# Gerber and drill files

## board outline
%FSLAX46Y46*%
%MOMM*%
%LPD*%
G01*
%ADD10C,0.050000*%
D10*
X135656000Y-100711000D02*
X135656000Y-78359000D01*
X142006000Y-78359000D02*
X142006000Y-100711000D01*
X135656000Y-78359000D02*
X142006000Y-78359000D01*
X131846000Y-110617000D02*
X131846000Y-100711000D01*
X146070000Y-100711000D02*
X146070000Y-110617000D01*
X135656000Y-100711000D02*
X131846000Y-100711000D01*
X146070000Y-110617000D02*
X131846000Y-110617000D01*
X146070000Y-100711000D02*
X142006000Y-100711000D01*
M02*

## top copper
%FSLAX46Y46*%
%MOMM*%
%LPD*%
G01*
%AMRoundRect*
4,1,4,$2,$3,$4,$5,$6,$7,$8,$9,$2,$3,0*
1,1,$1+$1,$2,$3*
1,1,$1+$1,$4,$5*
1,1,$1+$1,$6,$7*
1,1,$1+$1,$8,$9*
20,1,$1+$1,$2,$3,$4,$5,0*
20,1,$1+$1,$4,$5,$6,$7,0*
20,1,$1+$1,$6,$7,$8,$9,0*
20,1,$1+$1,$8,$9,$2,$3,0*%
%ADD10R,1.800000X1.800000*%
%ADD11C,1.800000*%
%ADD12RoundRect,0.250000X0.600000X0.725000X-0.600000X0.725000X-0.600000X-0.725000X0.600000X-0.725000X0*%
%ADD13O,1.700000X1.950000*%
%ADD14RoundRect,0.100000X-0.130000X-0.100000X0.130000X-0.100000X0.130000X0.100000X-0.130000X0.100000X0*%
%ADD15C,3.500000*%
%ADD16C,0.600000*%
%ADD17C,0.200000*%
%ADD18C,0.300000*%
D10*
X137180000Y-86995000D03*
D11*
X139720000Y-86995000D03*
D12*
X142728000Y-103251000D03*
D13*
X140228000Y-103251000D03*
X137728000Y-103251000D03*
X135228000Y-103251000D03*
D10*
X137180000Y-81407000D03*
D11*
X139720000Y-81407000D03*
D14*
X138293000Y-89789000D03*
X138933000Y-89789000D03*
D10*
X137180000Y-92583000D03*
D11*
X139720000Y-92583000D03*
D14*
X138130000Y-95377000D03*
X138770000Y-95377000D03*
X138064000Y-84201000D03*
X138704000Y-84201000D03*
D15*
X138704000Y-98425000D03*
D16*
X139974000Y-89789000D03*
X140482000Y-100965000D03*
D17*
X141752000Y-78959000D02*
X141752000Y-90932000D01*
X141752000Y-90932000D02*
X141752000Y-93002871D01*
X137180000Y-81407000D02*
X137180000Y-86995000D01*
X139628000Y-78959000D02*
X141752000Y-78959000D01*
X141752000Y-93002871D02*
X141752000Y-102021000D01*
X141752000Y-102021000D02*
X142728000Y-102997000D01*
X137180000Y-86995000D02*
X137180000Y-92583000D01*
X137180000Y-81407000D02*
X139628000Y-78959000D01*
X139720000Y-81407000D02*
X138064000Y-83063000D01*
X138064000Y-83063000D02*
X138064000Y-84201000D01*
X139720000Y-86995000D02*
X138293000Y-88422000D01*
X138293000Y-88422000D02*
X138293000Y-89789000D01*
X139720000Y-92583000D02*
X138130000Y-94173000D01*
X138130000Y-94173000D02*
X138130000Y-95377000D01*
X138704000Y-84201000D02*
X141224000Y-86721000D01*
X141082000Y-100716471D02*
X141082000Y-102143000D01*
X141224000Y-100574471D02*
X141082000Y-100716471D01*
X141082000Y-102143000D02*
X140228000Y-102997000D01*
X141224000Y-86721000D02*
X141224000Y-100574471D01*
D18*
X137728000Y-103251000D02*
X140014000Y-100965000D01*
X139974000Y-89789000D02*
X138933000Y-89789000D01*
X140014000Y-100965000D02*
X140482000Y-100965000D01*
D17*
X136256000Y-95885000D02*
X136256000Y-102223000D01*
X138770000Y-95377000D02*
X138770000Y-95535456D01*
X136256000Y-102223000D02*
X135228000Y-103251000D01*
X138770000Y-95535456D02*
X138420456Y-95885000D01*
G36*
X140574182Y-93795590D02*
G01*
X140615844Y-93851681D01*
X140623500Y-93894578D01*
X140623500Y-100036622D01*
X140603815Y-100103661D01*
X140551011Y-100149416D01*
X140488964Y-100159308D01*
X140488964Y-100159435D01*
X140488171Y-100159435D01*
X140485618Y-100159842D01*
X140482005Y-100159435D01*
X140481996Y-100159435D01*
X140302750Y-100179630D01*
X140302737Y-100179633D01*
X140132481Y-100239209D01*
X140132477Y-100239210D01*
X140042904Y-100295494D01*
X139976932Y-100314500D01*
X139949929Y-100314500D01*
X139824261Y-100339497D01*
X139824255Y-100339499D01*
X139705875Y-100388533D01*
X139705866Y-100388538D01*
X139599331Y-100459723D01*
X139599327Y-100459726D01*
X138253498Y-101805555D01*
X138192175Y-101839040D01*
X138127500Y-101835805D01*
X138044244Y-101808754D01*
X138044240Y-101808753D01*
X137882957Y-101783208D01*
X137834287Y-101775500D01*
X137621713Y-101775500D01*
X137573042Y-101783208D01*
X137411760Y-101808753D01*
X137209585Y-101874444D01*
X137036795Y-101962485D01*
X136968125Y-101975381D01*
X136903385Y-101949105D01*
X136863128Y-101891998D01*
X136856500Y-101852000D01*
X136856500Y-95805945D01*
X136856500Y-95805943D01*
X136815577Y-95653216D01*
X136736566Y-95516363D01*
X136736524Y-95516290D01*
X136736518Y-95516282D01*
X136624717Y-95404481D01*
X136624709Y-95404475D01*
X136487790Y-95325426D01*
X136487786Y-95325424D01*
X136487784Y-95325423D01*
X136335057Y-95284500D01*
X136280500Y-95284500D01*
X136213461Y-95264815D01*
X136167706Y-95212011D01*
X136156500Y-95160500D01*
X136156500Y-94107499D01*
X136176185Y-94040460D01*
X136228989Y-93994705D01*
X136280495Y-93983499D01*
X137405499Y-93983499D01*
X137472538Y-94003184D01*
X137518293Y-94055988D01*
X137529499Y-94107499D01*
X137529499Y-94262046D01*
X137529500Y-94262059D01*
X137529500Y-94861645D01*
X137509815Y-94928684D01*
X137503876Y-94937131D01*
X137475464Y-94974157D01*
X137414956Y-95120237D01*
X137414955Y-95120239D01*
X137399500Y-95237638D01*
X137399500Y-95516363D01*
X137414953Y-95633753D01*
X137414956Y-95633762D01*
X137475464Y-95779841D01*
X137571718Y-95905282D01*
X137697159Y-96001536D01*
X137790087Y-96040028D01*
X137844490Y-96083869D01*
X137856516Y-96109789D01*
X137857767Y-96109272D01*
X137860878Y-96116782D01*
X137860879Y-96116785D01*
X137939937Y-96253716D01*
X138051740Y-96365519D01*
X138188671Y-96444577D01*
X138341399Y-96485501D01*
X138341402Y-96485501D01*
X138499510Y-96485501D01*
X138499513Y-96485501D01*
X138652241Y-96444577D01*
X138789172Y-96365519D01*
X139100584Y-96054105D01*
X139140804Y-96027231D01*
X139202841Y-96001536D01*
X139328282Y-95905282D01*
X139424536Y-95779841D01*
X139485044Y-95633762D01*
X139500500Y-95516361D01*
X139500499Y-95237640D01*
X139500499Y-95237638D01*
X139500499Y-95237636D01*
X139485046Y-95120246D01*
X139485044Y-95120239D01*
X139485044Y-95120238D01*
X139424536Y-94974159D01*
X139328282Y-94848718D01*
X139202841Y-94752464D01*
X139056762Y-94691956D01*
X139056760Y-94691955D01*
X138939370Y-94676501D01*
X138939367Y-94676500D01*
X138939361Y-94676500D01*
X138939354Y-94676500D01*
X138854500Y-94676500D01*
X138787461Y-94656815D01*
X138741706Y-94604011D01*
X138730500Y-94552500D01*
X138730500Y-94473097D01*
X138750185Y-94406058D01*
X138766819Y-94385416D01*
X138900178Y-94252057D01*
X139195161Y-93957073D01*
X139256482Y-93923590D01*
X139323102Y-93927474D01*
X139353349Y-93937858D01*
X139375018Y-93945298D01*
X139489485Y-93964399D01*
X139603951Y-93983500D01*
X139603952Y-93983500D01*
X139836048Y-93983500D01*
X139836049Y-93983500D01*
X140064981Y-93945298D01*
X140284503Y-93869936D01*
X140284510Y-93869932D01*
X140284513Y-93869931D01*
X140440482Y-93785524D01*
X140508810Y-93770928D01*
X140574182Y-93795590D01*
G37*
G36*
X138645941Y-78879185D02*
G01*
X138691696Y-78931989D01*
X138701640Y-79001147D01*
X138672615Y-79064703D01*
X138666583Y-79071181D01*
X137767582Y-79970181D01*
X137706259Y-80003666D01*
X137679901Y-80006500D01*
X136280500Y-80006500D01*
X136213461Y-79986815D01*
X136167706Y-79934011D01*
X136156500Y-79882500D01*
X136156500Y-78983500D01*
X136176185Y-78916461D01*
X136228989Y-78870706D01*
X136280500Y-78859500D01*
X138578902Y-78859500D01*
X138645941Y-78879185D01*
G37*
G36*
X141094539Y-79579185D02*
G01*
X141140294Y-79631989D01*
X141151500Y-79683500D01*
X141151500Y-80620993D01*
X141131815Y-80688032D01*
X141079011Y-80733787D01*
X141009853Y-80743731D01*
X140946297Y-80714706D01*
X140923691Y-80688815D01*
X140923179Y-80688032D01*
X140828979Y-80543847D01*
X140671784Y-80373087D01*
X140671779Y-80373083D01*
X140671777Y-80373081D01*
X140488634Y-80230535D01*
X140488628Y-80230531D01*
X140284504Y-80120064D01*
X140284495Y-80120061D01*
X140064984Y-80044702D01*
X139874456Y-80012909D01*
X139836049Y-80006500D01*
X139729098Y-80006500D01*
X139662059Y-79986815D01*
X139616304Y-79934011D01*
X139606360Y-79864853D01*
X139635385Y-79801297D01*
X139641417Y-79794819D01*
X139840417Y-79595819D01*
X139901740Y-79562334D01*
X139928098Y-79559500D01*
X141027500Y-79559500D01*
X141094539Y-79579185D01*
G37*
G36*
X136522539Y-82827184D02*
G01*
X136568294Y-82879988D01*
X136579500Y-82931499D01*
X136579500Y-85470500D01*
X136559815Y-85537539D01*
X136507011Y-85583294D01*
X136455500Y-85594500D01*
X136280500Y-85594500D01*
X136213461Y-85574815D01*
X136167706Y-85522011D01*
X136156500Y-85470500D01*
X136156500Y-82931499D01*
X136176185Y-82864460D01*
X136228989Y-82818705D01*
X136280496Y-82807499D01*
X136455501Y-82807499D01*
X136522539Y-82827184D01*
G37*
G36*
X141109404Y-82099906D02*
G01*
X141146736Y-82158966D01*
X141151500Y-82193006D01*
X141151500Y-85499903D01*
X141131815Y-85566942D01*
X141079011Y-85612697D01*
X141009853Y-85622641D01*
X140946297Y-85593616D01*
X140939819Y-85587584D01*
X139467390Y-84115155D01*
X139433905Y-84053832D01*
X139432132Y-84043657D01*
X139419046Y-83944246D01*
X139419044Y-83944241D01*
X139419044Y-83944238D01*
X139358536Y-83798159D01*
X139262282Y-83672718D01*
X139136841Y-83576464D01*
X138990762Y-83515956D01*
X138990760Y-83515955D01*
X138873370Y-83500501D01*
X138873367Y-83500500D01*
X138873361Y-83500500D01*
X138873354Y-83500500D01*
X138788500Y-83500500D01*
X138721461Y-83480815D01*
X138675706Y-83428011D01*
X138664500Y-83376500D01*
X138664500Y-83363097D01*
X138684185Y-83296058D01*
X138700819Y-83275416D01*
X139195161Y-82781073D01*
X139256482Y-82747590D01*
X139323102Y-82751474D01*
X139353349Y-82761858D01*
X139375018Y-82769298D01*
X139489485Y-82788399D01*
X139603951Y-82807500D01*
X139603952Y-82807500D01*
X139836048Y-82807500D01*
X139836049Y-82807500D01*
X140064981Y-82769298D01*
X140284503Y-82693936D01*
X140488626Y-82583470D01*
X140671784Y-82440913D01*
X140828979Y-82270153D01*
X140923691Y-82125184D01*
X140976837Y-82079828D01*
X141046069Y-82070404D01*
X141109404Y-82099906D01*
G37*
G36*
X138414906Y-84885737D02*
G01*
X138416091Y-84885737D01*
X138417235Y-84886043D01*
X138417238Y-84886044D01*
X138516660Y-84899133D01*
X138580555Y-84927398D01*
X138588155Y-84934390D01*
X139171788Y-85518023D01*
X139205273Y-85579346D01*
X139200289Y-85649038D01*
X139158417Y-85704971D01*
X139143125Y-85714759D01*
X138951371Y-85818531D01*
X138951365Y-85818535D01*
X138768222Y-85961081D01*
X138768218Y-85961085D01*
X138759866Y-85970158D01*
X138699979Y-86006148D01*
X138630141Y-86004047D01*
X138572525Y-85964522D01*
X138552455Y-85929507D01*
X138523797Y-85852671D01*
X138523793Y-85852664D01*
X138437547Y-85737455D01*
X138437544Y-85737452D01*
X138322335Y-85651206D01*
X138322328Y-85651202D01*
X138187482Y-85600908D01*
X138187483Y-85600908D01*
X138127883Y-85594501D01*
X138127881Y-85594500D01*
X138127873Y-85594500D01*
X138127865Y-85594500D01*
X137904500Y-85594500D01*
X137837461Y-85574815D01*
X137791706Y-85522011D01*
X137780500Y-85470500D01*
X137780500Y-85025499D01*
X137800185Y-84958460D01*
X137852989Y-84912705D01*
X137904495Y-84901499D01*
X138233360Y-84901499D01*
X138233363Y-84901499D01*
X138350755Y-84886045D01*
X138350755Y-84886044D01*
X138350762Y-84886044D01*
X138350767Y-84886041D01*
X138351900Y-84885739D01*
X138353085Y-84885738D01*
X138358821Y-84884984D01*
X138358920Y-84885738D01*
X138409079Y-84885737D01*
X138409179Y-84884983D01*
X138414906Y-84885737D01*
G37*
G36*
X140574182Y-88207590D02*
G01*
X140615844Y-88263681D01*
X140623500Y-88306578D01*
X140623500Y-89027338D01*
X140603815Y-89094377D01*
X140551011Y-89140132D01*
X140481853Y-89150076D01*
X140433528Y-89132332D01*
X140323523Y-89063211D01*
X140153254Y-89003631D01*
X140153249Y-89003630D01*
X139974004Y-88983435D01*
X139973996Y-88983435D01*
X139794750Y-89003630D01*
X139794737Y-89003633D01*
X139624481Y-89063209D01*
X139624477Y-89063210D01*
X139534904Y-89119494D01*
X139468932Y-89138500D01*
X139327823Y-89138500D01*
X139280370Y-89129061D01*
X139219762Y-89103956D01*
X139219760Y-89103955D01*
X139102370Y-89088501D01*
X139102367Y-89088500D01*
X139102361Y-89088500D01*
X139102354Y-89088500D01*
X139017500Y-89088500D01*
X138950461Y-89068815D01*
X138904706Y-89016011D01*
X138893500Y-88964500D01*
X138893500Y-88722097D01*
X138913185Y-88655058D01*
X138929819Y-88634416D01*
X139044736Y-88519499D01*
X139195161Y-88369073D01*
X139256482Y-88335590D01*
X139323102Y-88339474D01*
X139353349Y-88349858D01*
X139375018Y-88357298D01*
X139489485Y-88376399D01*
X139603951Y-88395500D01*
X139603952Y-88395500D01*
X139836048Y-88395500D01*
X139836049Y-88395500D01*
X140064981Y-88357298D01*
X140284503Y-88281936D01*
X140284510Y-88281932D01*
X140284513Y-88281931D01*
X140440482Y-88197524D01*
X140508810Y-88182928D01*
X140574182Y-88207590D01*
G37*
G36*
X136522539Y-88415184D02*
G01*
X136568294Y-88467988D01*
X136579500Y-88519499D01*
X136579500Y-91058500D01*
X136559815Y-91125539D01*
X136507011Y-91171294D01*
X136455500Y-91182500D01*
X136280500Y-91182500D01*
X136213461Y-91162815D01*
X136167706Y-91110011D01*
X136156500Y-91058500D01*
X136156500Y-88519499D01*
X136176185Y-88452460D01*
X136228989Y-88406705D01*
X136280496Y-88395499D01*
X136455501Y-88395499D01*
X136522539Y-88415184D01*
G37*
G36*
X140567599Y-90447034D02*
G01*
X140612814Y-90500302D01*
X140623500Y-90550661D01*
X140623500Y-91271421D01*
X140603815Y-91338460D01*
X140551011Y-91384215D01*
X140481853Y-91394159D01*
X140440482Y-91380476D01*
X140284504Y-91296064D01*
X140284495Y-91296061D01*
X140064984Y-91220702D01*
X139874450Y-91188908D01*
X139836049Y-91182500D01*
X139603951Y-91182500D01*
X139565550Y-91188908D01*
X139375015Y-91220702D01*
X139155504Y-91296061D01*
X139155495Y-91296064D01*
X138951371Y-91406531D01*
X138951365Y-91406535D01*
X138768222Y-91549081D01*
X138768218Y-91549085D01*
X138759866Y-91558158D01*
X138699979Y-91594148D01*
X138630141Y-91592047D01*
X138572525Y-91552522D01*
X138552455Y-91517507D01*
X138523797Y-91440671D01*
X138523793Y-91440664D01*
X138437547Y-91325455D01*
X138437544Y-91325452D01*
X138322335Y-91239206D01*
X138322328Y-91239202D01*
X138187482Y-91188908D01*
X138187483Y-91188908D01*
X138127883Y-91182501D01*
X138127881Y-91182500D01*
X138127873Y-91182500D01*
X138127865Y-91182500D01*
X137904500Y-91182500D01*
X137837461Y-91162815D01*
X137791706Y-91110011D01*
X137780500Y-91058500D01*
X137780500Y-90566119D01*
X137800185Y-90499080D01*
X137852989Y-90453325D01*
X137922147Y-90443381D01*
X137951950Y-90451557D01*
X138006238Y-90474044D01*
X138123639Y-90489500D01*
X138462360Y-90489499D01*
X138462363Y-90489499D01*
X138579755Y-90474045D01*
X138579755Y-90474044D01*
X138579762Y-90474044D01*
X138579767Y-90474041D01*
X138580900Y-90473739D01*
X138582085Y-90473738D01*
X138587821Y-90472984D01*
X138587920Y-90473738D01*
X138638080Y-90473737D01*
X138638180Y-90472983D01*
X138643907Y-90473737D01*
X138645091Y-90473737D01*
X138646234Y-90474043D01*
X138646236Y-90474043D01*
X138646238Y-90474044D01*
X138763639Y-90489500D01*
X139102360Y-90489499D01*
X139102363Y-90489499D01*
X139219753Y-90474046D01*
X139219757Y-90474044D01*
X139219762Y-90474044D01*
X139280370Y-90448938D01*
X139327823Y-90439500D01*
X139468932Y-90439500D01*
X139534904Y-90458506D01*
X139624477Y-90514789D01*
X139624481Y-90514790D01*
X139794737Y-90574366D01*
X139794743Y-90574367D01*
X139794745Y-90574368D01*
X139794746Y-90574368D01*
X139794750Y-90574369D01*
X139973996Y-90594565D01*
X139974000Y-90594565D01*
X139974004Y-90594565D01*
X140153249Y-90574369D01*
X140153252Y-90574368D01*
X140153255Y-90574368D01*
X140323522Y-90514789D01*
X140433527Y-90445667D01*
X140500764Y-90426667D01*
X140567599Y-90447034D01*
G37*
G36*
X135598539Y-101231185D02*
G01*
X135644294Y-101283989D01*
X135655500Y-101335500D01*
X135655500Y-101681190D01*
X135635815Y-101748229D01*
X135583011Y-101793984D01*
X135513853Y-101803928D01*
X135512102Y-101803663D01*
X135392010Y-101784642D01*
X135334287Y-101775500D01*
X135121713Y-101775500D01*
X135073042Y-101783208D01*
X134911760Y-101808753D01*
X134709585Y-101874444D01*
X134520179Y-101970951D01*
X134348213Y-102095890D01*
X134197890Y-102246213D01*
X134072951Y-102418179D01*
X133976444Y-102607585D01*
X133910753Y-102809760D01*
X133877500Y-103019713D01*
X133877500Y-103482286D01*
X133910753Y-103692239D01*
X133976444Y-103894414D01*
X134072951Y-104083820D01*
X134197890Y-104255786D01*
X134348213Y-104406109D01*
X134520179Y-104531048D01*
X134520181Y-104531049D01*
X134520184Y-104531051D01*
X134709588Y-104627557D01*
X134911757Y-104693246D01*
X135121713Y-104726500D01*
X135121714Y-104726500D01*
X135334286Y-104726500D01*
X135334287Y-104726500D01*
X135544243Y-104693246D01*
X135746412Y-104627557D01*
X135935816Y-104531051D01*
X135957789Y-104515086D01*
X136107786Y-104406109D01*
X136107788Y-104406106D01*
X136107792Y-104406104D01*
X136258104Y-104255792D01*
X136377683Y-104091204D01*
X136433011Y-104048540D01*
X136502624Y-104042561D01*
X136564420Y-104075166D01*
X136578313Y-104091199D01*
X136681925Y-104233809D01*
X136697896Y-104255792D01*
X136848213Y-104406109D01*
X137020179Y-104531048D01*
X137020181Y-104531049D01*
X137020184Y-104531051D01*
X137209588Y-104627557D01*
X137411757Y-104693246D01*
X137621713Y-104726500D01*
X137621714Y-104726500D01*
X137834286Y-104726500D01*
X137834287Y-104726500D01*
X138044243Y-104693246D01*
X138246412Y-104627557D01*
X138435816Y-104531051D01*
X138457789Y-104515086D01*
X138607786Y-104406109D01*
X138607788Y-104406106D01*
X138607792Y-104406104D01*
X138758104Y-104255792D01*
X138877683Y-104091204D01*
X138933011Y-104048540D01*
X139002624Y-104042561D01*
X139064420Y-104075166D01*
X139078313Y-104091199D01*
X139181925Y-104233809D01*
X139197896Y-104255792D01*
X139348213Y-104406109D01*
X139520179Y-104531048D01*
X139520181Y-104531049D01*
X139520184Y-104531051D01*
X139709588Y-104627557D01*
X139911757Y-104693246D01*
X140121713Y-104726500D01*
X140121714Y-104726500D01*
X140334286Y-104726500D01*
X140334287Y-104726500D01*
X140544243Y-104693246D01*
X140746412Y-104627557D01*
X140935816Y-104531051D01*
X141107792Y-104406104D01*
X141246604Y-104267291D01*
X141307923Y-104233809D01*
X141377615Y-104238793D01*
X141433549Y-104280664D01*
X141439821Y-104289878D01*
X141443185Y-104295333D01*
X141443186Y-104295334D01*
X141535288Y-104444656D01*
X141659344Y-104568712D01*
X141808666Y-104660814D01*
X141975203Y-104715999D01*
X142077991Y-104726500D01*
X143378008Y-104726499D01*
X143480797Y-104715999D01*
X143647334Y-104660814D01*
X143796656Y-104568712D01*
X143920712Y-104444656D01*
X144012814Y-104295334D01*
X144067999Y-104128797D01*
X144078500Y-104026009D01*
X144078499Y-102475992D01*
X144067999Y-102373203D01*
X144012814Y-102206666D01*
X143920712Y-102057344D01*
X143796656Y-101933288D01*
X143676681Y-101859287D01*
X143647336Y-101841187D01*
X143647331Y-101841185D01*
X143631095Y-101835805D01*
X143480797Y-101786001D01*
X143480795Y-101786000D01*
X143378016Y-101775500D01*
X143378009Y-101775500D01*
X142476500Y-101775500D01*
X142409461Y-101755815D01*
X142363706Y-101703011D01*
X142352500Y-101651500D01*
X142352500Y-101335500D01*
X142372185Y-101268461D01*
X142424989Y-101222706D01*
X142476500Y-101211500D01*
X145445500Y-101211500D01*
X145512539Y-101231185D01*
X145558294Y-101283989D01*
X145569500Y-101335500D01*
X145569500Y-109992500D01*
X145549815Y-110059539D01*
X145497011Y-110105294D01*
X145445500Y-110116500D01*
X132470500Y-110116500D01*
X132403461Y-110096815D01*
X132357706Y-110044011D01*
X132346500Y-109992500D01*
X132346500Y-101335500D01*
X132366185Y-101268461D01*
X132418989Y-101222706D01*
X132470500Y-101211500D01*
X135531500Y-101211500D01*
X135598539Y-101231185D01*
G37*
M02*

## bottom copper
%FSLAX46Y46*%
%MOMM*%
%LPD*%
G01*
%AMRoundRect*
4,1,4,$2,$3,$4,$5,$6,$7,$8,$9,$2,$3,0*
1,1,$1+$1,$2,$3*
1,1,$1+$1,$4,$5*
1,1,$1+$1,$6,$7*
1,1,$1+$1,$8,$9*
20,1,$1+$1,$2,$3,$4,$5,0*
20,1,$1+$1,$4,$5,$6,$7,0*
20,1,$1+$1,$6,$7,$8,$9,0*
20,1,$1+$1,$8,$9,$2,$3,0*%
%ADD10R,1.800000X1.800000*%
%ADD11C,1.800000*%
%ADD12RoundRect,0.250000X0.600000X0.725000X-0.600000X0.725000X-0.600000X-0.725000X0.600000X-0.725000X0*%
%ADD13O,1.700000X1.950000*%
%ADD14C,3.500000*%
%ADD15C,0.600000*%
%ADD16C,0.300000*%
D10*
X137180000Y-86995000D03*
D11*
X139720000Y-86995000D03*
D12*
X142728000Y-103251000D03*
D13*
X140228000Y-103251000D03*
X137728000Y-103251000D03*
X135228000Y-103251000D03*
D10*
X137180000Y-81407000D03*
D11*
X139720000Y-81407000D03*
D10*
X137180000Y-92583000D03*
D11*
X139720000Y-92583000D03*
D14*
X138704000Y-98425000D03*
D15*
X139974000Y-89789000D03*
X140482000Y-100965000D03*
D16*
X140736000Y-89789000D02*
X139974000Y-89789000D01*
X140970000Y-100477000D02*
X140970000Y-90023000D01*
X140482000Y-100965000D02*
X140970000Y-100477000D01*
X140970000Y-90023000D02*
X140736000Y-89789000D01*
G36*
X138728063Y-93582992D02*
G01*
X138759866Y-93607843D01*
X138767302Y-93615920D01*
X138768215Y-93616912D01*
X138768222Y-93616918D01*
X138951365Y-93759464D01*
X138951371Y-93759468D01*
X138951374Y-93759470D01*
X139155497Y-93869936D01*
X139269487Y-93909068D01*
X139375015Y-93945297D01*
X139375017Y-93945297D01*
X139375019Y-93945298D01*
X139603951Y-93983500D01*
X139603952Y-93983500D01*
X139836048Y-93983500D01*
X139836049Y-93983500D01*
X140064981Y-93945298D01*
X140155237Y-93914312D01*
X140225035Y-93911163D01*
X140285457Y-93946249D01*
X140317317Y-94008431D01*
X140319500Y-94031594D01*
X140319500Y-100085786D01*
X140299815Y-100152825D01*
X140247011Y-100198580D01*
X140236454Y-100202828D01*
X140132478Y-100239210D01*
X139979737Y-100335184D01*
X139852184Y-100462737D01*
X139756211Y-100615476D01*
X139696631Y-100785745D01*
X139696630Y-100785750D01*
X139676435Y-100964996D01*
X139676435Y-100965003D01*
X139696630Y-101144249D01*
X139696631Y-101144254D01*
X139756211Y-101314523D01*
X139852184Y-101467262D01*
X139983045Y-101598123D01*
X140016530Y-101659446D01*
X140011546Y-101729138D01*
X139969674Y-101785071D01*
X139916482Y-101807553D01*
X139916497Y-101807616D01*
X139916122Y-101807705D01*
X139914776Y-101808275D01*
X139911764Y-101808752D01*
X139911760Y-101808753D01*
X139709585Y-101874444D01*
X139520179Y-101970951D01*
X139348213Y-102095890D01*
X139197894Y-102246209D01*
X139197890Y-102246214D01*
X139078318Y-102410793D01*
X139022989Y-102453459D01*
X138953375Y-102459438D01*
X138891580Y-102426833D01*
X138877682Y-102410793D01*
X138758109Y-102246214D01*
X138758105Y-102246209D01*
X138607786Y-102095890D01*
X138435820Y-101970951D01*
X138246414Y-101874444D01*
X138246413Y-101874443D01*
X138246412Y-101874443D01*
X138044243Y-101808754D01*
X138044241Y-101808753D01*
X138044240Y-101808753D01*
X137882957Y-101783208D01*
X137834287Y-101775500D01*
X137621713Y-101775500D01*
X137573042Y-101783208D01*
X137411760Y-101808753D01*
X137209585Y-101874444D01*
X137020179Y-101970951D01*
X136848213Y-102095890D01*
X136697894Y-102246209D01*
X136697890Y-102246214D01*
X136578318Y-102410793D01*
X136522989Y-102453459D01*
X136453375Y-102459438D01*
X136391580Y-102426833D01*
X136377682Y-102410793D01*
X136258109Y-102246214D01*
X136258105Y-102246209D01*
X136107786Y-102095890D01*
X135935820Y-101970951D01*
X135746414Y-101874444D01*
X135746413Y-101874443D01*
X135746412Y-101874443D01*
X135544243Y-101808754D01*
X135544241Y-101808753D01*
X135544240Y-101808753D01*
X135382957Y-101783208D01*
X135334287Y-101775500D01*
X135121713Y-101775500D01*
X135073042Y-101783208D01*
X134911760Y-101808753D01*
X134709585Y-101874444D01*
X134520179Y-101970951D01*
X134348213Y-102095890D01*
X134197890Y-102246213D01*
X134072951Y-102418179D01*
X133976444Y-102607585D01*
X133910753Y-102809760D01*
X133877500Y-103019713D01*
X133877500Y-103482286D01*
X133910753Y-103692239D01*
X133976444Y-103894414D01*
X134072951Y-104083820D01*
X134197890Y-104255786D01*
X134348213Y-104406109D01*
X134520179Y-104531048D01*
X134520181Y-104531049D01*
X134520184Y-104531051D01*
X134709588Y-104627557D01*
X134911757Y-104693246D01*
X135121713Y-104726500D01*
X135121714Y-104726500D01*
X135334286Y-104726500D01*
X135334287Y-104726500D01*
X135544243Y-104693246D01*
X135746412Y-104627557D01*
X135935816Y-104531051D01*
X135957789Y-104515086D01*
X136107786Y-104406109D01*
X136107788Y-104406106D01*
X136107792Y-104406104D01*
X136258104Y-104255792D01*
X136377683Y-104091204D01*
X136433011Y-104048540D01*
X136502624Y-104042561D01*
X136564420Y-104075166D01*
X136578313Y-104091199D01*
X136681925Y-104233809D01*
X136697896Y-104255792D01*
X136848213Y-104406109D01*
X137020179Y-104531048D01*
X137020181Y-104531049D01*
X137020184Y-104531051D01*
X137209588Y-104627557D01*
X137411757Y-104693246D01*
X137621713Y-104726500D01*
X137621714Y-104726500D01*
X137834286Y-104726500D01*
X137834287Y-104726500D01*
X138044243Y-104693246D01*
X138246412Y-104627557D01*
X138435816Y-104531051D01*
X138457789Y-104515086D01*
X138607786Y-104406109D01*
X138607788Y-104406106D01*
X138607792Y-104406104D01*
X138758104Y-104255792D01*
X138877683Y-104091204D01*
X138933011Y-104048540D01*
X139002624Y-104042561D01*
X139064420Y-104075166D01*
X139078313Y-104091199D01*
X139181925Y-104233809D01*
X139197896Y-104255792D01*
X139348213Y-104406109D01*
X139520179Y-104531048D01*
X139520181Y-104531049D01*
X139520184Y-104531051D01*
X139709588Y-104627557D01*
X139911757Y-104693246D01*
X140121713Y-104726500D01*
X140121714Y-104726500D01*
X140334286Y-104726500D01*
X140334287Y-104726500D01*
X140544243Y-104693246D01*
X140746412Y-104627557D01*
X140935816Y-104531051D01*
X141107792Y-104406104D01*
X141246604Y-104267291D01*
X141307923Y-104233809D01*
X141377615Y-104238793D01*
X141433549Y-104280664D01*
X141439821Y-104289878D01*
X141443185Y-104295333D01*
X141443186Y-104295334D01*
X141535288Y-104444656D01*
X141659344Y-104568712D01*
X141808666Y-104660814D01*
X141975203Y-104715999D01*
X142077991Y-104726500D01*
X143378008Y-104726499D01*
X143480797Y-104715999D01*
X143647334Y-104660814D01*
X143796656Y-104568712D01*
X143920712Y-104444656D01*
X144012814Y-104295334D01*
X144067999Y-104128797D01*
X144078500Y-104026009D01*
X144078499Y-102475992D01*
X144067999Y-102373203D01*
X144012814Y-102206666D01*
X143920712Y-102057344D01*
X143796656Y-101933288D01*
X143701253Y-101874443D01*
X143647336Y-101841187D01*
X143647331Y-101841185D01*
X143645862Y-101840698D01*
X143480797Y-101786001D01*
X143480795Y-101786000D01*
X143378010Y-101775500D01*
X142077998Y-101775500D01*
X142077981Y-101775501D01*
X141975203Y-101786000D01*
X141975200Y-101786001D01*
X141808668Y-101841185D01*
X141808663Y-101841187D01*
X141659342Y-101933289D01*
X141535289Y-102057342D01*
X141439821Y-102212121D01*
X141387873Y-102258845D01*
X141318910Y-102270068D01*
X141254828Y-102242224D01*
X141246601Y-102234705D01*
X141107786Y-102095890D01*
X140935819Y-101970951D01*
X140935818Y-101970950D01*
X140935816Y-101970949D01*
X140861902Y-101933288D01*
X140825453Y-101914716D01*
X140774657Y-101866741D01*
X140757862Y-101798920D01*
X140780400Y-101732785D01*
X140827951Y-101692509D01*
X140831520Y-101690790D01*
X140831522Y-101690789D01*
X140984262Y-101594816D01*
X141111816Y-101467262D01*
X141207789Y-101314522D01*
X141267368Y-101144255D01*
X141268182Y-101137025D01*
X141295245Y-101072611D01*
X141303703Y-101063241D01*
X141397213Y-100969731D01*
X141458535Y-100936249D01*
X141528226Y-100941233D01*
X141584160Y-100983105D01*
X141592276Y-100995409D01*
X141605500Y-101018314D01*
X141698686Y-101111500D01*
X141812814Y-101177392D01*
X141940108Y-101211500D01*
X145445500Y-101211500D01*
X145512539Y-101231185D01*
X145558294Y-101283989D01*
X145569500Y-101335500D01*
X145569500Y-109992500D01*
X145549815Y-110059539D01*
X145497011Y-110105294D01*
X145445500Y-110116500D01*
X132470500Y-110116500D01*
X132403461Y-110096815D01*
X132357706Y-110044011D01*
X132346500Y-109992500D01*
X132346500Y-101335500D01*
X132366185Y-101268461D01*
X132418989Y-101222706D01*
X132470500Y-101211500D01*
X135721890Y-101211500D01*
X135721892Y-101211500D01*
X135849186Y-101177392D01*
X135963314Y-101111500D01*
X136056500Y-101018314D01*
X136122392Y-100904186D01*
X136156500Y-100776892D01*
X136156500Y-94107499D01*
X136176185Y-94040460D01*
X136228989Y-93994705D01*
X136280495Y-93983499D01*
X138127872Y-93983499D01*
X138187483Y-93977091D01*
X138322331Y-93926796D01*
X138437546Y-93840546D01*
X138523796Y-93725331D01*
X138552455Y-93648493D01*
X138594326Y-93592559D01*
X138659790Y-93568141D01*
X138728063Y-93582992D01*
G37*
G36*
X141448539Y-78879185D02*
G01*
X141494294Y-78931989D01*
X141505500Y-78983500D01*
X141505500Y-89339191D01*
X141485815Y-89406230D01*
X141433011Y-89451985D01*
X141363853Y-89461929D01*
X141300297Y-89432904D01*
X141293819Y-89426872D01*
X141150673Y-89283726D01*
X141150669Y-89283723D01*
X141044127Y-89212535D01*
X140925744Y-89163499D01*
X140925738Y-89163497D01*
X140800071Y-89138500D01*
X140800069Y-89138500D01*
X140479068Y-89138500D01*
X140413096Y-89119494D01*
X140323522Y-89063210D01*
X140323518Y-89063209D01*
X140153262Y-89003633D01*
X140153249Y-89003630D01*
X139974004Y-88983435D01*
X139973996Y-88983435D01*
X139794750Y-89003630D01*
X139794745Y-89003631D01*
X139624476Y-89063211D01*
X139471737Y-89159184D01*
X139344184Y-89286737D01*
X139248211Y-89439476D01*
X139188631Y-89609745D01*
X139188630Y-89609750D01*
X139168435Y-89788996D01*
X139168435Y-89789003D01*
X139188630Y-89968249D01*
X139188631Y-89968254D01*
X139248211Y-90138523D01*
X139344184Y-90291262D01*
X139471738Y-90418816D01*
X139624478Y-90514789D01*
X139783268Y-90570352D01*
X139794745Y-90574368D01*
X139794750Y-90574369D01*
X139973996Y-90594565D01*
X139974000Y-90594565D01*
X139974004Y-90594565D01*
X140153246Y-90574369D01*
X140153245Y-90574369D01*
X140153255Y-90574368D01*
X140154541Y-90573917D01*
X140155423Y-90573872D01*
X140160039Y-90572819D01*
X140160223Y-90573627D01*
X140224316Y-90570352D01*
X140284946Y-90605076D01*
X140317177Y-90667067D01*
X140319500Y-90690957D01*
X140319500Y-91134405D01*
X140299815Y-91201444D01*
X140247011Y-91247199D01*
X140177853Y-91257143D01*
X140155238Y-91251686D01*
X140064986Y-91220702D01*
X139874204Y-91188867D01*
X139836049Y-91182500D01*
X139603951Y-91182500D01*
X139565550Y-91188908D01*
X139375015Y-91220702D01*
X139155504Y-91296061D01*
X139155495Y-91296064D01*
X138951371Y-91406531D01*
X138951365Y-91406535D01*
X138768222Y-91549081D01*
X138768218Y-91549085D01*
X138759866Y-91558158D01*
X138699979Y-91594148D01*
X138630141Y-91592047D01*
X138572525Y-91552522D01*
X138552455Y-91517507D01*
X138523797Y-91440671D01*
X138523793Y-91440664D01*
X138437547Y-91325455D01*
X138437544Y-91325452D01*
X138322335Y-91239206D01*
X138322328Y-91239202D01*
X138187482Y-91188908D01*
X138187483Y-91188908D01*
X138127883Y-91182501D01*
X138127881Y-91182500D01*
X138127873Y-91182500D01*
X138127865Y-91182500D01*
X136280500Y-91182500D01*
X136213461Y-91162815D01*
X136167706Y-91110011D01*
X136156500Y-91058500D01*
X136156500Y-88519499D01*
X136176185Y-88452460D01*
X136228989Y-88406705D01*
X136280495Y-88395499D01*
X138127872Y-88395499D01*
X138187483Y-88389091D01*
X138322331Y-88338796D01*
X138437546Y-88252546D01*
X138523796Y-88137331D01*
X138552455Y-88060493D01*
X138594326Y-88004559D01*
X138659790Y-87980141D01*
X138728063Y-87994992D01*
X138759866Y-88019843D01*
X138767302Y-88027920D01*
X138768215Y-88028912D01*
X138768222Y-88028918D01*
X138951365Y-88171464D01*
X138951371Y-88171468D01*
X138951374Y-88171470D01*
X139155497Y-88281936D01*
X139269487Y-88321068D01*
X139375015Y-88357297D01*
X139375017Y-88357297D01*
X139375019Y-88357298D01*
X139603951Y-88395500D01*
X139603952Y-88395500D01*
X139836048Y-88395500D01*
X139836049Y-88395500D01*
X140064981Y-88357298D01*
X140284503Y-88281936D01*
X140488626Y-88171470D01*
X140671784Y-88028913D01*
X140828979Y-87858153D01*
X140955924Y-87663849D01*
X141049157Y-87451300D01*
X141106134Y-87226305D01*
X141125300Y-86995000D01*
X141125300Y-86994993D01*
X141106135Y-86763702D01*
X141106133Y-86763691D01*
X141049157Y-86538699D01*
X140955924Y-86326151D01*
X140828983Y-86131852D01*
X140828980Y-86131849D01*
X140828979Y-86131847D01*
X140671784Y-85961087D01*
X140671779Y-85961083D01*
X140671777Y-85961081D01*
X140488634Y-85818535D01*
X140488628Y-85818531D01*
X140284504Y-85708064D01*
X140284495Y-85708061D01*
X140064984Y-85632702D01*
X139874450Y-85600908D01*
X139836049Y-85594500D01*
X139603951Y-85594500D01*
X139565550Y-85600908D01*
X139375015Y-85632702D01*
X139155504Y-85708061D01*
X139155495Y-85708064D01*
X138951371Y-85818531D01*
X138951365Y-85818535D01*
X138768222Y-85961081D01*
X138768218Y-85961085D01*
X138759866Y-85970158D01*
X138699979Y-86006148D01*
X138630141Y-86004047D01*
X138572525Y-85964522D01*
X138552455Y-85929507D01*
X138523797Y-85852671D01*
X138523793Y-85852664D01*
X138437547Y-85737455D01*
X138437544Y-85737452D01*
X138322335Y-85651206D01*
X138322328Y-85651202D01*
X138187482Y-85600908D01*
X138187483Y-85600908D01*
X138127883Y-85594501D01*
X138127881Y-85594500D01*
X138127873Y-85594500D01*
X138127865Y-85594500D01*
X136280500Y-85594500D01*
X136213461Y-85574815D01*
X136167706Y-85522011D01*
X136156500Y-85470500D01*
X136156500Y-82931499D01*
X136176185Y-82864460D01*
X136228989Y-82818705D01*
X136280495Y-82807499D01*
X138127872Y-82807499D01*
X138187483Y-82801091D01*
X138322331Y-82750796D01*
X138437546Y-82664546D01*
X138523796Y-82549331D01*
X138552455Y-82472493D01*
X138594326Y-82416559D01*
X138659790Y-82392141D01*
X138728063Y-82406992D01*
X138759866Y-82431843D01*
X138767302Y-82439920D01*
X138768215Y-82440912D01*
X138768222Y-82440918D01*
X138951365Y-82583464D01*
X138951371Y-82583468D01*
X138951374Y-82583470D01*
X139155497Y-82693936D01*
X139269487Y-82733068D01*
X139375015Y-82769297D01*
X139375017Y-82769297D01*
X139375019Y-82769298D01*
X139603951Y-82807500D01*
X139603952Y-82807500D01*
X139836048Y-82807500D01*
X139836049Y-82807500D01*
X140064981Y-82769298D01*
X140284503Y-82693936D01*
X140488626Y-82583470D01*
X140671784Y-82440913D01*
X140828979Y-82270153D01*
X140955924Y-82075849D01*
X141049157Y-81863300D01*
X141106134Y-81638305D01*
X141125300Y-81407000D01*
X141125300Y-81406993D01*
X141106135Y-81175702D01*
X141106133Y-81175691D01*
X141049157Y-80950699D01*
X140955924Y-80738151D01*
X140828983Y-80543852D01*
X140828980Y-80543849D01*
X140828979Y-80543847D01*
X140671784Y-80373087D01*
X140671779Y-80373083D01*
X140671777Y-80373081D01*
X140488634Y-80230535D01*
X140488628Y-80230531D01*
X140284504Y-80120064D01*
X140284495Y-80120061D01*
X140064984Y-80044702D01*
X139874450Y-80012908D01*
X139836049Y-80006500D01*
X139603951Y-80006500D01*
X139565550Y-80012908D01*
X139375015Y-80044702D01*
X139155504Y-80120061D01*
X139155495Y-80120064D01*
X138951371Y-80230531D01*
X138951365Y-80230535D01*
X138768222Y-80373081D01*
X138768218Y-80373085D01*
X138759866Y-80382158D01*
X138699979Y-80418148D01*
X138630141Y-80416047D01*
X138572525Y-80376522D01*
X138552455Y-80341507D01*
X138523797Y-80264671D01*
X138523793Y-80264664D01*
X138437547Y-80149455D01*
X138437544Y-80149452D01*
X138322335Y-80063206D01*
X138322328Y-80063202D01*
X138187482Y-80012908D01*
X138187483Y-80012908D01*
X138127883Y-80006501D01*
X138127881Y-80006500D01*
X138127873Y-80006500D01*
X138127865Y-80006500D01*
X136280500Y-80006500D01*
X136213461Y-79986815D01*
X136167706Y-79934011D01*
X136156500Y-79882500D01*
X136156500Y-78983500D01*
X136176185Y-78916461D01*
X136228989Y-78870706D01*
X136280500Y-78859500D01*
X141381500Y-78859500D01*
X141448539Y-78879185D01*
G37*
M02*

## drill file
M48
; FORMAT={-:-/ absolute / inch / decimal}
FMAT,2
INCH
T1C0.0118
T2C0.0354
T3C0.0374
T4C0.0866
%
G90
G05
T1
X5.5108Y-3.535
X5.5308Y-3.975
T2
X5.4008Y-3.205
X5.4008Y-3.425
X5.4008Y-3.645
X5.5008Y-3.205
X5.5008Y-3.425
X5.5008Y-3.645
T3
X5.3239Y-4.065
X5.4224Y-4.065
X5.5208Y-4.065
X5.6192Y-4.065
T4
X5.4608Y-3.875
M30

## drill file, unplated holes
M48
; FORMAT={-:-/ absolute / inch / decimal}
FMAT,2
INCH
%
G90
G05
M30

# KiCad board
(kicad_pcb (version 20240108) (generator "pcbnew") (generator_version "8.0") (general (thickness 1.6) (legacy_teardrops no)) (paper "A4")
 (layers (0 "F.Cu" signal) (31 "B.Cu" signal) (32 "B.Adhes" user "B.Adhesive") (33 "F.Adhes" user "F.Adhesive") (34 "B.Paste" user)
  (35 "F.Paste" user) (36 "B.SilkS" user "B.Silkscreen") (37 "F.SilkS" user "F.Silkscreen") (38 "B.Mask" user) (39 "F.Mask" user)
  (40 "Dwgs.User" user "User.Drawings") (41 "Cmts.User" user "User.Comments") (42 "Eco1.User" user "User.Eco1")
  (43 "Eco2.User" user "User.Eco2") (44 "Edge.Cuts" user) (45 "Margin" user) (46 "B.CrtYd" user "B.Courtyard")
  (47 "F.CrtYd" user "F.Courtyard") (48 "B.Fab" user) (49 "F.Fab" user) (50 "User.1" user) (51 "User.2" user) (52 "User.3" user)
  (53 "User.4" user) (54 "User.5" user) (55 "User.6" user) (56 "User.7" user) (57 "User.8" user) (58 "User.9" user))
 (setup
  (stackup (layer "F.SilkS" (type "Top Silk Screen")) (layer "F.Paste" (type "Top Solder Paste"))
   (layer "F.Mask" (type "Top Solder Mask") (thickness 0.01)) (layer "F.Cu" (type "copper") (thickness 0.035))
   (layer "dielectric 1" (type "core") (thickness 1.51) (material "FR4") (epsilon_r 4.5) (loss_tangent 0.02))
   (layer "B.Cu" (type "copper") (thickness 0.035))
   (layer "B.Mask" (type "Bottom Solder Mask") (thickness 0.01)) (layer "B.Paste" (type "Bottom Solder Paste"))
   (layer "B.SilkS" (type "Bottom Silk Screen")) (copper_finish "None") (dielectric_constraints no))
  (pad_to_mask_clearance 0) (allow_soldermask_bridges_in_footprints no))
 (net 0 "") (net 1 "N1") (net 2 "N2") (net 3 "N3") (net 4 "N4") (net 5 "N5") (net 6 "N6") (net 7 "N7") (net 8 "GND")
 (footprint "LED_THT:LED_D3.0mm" (layer "F.Cu") (at 137.18 86.995)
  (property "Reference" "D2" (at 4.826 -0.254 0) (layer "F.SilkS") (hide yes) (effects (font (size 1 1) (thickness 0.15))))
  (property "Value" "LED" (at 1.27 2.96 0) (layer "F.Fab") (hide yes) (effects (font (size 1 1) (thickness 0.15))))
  (pad "1" thru_hole rect (at 0 0) (size 1.8 1.8) (drill 0.9) (layers "*.Cu" "*.Mask") (remove_unused_layers no) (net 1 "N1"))
  (pad "2" thru_hole circle (at 2.54 0) (size 1.8 1.8) (drill 0.9) (layers "*.Cu" "*.Mask") (remove_unused_layers no) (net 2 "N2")))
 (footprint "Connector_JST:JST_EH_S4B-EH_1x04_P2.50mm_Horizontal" (layer "F.Cu") (at 142.728 103.251 180)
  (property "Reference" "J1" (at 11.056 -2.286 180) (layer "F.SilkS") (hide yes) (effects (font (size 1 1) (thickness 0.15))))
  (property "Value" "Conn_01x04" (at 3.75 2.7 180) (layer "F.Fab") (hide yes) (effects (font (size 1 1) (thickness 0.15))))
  (pad "1" thru_hole roundrect (at 0 0 180) (size 1.7 1.95) (drill 0.95) (layers "*.Cu" "*.Mask") (remove_unused_layers no)
   (roundrect_rratio 0.147059) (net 1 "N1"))
  (pad "2" thru_hole oval (at 2.5 0 180) (size 1.7 1.95) (drill 0.95) (layers "*.Cu" "*.Mask") (remove_unused_layers no) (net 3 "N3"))
  (pad "3" thru_hole oval (at 5 0 180) (size 1.7 1.95) (drill 0.95) (layers "*.Cu" "*.Mask") (remove_unused_layers no) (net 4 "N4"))
  (pad "4" thru_hole oval (at 7.5 0 180) (size 1.7 1.95) (drill 0.95) (layers "*.Cu" "*.Mask") (remove_unused_layers no) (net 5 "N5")))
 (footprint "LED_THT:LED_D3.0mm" (layer "F.Cu") (at 137.18 81.407)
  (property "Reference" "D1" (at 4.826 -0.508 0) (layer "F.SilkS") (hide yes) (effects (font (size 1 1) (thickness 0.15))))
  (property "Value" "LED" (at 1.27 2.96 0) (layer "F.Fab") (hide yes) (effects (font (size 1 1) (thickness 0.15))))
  (pad "1" thru_hole rect (at 0 0) (size 1.8 1.8) (drill 0.9) (layers "*.Cu" "*.Mask") (remove_unused_layers no) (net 1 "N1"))
  (pad "2" thru_hole circle (at 2.54 0) (size 1.8 1.8) (drill 0.9) (layers "*.Cu" "*.Mask") (remove_unused_layers no) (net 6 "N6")))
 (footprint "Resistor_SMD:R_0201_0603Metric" (layer "F.Cu") (at 138.613 89.789)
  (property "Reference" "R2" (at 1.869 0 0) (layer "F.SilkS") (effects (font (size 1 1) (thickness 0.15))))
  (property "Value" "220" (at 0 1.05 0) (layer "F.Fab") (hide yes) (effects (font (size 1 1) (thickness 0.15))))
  (pad "" smd roundrect (at -0.345 0) (size 0.318 0.36) (layers "F.Paste") (roundrect_rratio 0.25))
  (pad "" smd roundrect (at 0.345 0) (size 0.318 0.36) (layers "F.Paste") (roundrect_rratio 0.25))
  (pad "1" smd roundrect (at -0.32 0) (size 0.46 0.4) (layers "F.Cu" "F.Mask") (roundrect_rratio 0.25) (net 2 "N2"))
  (pad "2" smd roundrect (at 0.32 0) (size 0.46 0.4) (layers "F.Cu" "F.Mask") (roundrect_rratio 0.25) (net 4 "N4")))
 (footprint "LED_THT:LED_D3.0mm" (layer "F.Cu") (at 137.18 92.583)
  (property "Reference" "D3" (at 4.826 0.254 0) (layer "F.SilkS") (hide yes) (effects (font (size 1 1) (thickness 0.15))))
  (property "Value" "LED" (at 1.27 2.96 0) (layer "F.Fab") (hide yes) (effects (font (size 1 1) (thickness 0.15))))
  (pad "1" thru_hole rect (at 0 0) (size 1.8 1.8) (drill 0.9) (layers "*.Cu" "*.Mask") (remove_unused_layers no) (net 1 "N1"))
  (pad "2" thru_hole circle (at 2.54 0) (size 1.8 1.8) (drill 0.9) (layers "*.Cu" "*.Mask") (remove_unused_layers no) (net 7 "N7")))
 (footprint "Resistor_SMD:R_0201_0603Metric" (layer "F.Cu") (at 138.45 95.377)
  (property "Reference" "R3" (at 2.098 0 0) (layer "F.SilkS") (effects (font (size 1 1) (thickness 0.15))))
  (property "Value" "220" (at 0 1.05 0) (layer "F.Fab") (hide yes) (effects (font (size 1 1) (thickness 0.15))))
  (pad "" smd roundrect (at -0.345 0) (size 0.318 0.36) (layers "F.Paste") (roundrect_rratio 0.25))
  (pad "" smd roundrect (at 0.345 0) (size 0.318 0.36) (layers "F.Paste") (roundrect_rratio 0.25))
  (pad "1" smd roundrect (at -0.32 0) (size 0.46 0.4) (layers "F.Cu" "F.Mask") (roundrect_rratio 0.25) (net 7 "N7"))
  (pad "2" smd roundrect (at 0.32 0) (size 0.46 0.4) (layers "F.Cu" "F.Mask") (roundrect_rratio 0.25) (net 5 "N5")))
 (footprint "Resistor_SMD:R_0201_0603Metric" (layer "F.Cu") (at 138.384 84.201)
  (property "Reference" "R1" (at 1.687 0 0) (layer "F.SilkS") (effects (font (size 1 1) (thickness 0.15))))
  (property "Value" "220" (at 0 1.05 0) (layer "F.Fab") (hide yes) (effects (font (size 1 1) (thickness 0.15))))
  (pad "" smd roundrect (at -0.345 0) (size 0.318 0.36) (layers "F.Paste") (roundrect_rratio 0.25))
  (pad "" smd roundrect (at 0.345 0) (size 0.318 0.36) (layers "F.Paste") (roundrect_rratio 0.25))
  (pad "1" smd roundrect (at -0.32 0) (size 0.46 0.4) (layers "F.Cu" "F.Mask") (roundrect_rratio 0.25) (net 6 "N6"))
  (pad "2" smd roundrect (at 0.32 0) (size 0.46 0.4) (layers "F.Cu" "F.Mask") (roundrect_rratio 0.25) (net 3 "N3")))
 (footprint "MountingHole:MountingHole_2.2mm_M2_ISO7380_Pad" (layer "F.Cu") (at 138.704 98.425)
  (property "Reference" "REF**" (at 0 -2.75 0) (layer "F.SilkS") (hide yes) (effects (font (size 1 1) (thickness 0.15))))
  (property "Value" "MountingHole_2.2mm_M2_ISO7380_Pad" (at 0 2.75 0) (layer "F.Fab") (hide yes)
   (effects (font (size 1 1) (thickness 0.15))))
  (pad "1" thru_hole circle (at 0 0) (size 3.5 3.5) (drill 2.2) (layers "*.Cu" "*.Mask") (remove_unused_layers no) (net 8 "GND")))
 (gr_line (start 135.656 100.711) (end 135.656 78.359) (stroke (width 0.05) (type default)) (layer "Edge.Cuts"))
 (gr_line (start 142.006 78.359) (end 142.006 100.711) (stroke (width 0.05) (type default)) (layer "Edge.Cuts"))
 (gr_line (start 135.656 78.359) (end 142.006 78.359) (stroke (width 0.05) (type default)) (layer "Edge.Cuts"))
 (gr_line (start 131.846 110.617) (end 131.846 100.711) (stroke (width 0.05) (type default)) (layer "Edge.Cuts"))
 (gr_line (start 146.07 100.711) (end 146.07 110.617) (stroke (width 0.05) (type default)) (layer "Edge.Cuts"))
 (gr_line (start 135.656 100.711) (end 131.846 100.711) (stroke (width 0.05) (type default)) (layer "Edge.Cuts"))
 (gr_line (start 146.07 110.617) (end 131.846 110.617) (stroke (width 0.05) (type default)) (layer "Edge.Cuts"))
 (gr_line (start 146.07 100.711) (end 142.006 100.711) (stroke (width 0.05) (type default)) (layer "Edge.Cuts"))
 (segment (start 141.752 78.959) (end 141.752 90.932) (width 0.2) (layer "F.Cu") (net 1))
 (segment (start 141.752 90.932) (end 141.752 93.002871) (width 0.2) (layer "F.Cu") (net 1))
 (segment (start 137.18 81.407) (end 137.18 86.995) (width 0.2) (layer "F.Cu") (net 1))
 (segment (start 139.628 78.959) (end 141.752 78.959) (width 0.2) (layer "F.Cu") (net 1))
 (segment (start 141.752 93.002871) (end 141.752 102.021) (width 0.2) (layer "F.Cu") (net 1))
 (segment (start 141.752 102.021) (end 142.728 102.997) (width 0.2) (layer "F.Cu") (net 1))
 (segment (start 137.18 86.995) (end 137.18 92.583) (width 0.2) (layer "F.Cu") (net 1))
 (segment (start 137.18 81.407) (end 139.628 78.959) (width 0.2) (layer "F.Cu") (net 1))
 (segment (start 139.72 81.407) (end 138.064 83.063) (width 0.2) (layer "F.Cu") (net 6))
 (segment (start 138.064 83.063) (end 138.064 84.201) (width 0.2) (layer "F.Cu") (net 6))
 (segment (start 139.72 86.995) (end 138.293 88.422) (width 0.2) (layer "F.Cu") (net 2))
 (segment (start 138.293 88.422) (end 138.293 89.789) (width 0.2) (layer "F.Cu") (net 2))
 (segment (start 139.72 92.583) (end 138.13 94.173) (width 0.2) (layer "F.Cu") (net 7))
 (segment (start 138.13 94.173) (end 138.13 95.377) (width 0.2) (layer "F.Cu") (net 7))
 (segment (start 138.704 84.201) (end 141.224 86.721) (width 0.2) (layer "F.Cu") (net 3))
 (segment (start 141.082 100.716471) (end 141.082 102.143) (width 0.2) (layer "F.Cu") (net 3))
 (segment (start 141.224 100.574471) (end 141.082 100.716471) (width 0.2) (layer "F.Cu") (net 3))
 (segment (start 141.082 102.143) (end 140.228 102.997) (width 0.2) (layer "F.Cu") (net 3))
 (segment (start 141.224 86.721) (end 141.224 100.574471) (width 0.2) (layer "F.Cu") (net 3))
 (segment (start 137.728 103.251) (end 140.014 100.965) (width 0.3) (layer "F.Cu") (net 4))
 (segment (start 139.974 89.789) (end 138.933 89.789) (width 0.3) (layer "F.Cu") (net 4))
 (segment (start 140.014 100.965) (end 140.482 100.965) (width 0.3) (layer "F.Cu") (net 4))
 (via (at 139.974 89.789) (size 0.6) (drill 0.3) (layers "F.Cu" "B.Cu") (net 4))
 (via (at 140.482 100.965) (size 0.6) (drill 0.3) (layers "F.Cu" "B.Cu") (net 4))
 (segment (start 140.736 89.789) (end 139.974 89.789) (width 0.3) (layer "B.Cu") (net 4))
 (segment (start 140.97 100.477) (end 140.97 90.023) (width 0.3) (layer "B.Cu") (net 4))
 (segment (start 140.482 100.965) (end 140.97 100.477) (width 0.3) (layer "B.Cu") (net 4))
 (segment (start 140.97 90.023) (end 140.736 89.789) (width 0.3) (layer "B.Cu") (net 4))
 (segment (start 136.256 95.885) (end 136.256 102.223) (width 0.2) (layer "F.Cu") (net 5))
 (segment (start 138.77 95.377) (end 138.77 95.535456) (width 0.2) (layer "F.Cu") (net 5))
 (segment (start 136.256 102.223) (end 135.228 103.251) (width 0.2) (layer "F.Cu") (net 5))
 (segment (start 138.77 95.535456) (end 138.420456 95.885) (width 0.2) (layer "F.Cu") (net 5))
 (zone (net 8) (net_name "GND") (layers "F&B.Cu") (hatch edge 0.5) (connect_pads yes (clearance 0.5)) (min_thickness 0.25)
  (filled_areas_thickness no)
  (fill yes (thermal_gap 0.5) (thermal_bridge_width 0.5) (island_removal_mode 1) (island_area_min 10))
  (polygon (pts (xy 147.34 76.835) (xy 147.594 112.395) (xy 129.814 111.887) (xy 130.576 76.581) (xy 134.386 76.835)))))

